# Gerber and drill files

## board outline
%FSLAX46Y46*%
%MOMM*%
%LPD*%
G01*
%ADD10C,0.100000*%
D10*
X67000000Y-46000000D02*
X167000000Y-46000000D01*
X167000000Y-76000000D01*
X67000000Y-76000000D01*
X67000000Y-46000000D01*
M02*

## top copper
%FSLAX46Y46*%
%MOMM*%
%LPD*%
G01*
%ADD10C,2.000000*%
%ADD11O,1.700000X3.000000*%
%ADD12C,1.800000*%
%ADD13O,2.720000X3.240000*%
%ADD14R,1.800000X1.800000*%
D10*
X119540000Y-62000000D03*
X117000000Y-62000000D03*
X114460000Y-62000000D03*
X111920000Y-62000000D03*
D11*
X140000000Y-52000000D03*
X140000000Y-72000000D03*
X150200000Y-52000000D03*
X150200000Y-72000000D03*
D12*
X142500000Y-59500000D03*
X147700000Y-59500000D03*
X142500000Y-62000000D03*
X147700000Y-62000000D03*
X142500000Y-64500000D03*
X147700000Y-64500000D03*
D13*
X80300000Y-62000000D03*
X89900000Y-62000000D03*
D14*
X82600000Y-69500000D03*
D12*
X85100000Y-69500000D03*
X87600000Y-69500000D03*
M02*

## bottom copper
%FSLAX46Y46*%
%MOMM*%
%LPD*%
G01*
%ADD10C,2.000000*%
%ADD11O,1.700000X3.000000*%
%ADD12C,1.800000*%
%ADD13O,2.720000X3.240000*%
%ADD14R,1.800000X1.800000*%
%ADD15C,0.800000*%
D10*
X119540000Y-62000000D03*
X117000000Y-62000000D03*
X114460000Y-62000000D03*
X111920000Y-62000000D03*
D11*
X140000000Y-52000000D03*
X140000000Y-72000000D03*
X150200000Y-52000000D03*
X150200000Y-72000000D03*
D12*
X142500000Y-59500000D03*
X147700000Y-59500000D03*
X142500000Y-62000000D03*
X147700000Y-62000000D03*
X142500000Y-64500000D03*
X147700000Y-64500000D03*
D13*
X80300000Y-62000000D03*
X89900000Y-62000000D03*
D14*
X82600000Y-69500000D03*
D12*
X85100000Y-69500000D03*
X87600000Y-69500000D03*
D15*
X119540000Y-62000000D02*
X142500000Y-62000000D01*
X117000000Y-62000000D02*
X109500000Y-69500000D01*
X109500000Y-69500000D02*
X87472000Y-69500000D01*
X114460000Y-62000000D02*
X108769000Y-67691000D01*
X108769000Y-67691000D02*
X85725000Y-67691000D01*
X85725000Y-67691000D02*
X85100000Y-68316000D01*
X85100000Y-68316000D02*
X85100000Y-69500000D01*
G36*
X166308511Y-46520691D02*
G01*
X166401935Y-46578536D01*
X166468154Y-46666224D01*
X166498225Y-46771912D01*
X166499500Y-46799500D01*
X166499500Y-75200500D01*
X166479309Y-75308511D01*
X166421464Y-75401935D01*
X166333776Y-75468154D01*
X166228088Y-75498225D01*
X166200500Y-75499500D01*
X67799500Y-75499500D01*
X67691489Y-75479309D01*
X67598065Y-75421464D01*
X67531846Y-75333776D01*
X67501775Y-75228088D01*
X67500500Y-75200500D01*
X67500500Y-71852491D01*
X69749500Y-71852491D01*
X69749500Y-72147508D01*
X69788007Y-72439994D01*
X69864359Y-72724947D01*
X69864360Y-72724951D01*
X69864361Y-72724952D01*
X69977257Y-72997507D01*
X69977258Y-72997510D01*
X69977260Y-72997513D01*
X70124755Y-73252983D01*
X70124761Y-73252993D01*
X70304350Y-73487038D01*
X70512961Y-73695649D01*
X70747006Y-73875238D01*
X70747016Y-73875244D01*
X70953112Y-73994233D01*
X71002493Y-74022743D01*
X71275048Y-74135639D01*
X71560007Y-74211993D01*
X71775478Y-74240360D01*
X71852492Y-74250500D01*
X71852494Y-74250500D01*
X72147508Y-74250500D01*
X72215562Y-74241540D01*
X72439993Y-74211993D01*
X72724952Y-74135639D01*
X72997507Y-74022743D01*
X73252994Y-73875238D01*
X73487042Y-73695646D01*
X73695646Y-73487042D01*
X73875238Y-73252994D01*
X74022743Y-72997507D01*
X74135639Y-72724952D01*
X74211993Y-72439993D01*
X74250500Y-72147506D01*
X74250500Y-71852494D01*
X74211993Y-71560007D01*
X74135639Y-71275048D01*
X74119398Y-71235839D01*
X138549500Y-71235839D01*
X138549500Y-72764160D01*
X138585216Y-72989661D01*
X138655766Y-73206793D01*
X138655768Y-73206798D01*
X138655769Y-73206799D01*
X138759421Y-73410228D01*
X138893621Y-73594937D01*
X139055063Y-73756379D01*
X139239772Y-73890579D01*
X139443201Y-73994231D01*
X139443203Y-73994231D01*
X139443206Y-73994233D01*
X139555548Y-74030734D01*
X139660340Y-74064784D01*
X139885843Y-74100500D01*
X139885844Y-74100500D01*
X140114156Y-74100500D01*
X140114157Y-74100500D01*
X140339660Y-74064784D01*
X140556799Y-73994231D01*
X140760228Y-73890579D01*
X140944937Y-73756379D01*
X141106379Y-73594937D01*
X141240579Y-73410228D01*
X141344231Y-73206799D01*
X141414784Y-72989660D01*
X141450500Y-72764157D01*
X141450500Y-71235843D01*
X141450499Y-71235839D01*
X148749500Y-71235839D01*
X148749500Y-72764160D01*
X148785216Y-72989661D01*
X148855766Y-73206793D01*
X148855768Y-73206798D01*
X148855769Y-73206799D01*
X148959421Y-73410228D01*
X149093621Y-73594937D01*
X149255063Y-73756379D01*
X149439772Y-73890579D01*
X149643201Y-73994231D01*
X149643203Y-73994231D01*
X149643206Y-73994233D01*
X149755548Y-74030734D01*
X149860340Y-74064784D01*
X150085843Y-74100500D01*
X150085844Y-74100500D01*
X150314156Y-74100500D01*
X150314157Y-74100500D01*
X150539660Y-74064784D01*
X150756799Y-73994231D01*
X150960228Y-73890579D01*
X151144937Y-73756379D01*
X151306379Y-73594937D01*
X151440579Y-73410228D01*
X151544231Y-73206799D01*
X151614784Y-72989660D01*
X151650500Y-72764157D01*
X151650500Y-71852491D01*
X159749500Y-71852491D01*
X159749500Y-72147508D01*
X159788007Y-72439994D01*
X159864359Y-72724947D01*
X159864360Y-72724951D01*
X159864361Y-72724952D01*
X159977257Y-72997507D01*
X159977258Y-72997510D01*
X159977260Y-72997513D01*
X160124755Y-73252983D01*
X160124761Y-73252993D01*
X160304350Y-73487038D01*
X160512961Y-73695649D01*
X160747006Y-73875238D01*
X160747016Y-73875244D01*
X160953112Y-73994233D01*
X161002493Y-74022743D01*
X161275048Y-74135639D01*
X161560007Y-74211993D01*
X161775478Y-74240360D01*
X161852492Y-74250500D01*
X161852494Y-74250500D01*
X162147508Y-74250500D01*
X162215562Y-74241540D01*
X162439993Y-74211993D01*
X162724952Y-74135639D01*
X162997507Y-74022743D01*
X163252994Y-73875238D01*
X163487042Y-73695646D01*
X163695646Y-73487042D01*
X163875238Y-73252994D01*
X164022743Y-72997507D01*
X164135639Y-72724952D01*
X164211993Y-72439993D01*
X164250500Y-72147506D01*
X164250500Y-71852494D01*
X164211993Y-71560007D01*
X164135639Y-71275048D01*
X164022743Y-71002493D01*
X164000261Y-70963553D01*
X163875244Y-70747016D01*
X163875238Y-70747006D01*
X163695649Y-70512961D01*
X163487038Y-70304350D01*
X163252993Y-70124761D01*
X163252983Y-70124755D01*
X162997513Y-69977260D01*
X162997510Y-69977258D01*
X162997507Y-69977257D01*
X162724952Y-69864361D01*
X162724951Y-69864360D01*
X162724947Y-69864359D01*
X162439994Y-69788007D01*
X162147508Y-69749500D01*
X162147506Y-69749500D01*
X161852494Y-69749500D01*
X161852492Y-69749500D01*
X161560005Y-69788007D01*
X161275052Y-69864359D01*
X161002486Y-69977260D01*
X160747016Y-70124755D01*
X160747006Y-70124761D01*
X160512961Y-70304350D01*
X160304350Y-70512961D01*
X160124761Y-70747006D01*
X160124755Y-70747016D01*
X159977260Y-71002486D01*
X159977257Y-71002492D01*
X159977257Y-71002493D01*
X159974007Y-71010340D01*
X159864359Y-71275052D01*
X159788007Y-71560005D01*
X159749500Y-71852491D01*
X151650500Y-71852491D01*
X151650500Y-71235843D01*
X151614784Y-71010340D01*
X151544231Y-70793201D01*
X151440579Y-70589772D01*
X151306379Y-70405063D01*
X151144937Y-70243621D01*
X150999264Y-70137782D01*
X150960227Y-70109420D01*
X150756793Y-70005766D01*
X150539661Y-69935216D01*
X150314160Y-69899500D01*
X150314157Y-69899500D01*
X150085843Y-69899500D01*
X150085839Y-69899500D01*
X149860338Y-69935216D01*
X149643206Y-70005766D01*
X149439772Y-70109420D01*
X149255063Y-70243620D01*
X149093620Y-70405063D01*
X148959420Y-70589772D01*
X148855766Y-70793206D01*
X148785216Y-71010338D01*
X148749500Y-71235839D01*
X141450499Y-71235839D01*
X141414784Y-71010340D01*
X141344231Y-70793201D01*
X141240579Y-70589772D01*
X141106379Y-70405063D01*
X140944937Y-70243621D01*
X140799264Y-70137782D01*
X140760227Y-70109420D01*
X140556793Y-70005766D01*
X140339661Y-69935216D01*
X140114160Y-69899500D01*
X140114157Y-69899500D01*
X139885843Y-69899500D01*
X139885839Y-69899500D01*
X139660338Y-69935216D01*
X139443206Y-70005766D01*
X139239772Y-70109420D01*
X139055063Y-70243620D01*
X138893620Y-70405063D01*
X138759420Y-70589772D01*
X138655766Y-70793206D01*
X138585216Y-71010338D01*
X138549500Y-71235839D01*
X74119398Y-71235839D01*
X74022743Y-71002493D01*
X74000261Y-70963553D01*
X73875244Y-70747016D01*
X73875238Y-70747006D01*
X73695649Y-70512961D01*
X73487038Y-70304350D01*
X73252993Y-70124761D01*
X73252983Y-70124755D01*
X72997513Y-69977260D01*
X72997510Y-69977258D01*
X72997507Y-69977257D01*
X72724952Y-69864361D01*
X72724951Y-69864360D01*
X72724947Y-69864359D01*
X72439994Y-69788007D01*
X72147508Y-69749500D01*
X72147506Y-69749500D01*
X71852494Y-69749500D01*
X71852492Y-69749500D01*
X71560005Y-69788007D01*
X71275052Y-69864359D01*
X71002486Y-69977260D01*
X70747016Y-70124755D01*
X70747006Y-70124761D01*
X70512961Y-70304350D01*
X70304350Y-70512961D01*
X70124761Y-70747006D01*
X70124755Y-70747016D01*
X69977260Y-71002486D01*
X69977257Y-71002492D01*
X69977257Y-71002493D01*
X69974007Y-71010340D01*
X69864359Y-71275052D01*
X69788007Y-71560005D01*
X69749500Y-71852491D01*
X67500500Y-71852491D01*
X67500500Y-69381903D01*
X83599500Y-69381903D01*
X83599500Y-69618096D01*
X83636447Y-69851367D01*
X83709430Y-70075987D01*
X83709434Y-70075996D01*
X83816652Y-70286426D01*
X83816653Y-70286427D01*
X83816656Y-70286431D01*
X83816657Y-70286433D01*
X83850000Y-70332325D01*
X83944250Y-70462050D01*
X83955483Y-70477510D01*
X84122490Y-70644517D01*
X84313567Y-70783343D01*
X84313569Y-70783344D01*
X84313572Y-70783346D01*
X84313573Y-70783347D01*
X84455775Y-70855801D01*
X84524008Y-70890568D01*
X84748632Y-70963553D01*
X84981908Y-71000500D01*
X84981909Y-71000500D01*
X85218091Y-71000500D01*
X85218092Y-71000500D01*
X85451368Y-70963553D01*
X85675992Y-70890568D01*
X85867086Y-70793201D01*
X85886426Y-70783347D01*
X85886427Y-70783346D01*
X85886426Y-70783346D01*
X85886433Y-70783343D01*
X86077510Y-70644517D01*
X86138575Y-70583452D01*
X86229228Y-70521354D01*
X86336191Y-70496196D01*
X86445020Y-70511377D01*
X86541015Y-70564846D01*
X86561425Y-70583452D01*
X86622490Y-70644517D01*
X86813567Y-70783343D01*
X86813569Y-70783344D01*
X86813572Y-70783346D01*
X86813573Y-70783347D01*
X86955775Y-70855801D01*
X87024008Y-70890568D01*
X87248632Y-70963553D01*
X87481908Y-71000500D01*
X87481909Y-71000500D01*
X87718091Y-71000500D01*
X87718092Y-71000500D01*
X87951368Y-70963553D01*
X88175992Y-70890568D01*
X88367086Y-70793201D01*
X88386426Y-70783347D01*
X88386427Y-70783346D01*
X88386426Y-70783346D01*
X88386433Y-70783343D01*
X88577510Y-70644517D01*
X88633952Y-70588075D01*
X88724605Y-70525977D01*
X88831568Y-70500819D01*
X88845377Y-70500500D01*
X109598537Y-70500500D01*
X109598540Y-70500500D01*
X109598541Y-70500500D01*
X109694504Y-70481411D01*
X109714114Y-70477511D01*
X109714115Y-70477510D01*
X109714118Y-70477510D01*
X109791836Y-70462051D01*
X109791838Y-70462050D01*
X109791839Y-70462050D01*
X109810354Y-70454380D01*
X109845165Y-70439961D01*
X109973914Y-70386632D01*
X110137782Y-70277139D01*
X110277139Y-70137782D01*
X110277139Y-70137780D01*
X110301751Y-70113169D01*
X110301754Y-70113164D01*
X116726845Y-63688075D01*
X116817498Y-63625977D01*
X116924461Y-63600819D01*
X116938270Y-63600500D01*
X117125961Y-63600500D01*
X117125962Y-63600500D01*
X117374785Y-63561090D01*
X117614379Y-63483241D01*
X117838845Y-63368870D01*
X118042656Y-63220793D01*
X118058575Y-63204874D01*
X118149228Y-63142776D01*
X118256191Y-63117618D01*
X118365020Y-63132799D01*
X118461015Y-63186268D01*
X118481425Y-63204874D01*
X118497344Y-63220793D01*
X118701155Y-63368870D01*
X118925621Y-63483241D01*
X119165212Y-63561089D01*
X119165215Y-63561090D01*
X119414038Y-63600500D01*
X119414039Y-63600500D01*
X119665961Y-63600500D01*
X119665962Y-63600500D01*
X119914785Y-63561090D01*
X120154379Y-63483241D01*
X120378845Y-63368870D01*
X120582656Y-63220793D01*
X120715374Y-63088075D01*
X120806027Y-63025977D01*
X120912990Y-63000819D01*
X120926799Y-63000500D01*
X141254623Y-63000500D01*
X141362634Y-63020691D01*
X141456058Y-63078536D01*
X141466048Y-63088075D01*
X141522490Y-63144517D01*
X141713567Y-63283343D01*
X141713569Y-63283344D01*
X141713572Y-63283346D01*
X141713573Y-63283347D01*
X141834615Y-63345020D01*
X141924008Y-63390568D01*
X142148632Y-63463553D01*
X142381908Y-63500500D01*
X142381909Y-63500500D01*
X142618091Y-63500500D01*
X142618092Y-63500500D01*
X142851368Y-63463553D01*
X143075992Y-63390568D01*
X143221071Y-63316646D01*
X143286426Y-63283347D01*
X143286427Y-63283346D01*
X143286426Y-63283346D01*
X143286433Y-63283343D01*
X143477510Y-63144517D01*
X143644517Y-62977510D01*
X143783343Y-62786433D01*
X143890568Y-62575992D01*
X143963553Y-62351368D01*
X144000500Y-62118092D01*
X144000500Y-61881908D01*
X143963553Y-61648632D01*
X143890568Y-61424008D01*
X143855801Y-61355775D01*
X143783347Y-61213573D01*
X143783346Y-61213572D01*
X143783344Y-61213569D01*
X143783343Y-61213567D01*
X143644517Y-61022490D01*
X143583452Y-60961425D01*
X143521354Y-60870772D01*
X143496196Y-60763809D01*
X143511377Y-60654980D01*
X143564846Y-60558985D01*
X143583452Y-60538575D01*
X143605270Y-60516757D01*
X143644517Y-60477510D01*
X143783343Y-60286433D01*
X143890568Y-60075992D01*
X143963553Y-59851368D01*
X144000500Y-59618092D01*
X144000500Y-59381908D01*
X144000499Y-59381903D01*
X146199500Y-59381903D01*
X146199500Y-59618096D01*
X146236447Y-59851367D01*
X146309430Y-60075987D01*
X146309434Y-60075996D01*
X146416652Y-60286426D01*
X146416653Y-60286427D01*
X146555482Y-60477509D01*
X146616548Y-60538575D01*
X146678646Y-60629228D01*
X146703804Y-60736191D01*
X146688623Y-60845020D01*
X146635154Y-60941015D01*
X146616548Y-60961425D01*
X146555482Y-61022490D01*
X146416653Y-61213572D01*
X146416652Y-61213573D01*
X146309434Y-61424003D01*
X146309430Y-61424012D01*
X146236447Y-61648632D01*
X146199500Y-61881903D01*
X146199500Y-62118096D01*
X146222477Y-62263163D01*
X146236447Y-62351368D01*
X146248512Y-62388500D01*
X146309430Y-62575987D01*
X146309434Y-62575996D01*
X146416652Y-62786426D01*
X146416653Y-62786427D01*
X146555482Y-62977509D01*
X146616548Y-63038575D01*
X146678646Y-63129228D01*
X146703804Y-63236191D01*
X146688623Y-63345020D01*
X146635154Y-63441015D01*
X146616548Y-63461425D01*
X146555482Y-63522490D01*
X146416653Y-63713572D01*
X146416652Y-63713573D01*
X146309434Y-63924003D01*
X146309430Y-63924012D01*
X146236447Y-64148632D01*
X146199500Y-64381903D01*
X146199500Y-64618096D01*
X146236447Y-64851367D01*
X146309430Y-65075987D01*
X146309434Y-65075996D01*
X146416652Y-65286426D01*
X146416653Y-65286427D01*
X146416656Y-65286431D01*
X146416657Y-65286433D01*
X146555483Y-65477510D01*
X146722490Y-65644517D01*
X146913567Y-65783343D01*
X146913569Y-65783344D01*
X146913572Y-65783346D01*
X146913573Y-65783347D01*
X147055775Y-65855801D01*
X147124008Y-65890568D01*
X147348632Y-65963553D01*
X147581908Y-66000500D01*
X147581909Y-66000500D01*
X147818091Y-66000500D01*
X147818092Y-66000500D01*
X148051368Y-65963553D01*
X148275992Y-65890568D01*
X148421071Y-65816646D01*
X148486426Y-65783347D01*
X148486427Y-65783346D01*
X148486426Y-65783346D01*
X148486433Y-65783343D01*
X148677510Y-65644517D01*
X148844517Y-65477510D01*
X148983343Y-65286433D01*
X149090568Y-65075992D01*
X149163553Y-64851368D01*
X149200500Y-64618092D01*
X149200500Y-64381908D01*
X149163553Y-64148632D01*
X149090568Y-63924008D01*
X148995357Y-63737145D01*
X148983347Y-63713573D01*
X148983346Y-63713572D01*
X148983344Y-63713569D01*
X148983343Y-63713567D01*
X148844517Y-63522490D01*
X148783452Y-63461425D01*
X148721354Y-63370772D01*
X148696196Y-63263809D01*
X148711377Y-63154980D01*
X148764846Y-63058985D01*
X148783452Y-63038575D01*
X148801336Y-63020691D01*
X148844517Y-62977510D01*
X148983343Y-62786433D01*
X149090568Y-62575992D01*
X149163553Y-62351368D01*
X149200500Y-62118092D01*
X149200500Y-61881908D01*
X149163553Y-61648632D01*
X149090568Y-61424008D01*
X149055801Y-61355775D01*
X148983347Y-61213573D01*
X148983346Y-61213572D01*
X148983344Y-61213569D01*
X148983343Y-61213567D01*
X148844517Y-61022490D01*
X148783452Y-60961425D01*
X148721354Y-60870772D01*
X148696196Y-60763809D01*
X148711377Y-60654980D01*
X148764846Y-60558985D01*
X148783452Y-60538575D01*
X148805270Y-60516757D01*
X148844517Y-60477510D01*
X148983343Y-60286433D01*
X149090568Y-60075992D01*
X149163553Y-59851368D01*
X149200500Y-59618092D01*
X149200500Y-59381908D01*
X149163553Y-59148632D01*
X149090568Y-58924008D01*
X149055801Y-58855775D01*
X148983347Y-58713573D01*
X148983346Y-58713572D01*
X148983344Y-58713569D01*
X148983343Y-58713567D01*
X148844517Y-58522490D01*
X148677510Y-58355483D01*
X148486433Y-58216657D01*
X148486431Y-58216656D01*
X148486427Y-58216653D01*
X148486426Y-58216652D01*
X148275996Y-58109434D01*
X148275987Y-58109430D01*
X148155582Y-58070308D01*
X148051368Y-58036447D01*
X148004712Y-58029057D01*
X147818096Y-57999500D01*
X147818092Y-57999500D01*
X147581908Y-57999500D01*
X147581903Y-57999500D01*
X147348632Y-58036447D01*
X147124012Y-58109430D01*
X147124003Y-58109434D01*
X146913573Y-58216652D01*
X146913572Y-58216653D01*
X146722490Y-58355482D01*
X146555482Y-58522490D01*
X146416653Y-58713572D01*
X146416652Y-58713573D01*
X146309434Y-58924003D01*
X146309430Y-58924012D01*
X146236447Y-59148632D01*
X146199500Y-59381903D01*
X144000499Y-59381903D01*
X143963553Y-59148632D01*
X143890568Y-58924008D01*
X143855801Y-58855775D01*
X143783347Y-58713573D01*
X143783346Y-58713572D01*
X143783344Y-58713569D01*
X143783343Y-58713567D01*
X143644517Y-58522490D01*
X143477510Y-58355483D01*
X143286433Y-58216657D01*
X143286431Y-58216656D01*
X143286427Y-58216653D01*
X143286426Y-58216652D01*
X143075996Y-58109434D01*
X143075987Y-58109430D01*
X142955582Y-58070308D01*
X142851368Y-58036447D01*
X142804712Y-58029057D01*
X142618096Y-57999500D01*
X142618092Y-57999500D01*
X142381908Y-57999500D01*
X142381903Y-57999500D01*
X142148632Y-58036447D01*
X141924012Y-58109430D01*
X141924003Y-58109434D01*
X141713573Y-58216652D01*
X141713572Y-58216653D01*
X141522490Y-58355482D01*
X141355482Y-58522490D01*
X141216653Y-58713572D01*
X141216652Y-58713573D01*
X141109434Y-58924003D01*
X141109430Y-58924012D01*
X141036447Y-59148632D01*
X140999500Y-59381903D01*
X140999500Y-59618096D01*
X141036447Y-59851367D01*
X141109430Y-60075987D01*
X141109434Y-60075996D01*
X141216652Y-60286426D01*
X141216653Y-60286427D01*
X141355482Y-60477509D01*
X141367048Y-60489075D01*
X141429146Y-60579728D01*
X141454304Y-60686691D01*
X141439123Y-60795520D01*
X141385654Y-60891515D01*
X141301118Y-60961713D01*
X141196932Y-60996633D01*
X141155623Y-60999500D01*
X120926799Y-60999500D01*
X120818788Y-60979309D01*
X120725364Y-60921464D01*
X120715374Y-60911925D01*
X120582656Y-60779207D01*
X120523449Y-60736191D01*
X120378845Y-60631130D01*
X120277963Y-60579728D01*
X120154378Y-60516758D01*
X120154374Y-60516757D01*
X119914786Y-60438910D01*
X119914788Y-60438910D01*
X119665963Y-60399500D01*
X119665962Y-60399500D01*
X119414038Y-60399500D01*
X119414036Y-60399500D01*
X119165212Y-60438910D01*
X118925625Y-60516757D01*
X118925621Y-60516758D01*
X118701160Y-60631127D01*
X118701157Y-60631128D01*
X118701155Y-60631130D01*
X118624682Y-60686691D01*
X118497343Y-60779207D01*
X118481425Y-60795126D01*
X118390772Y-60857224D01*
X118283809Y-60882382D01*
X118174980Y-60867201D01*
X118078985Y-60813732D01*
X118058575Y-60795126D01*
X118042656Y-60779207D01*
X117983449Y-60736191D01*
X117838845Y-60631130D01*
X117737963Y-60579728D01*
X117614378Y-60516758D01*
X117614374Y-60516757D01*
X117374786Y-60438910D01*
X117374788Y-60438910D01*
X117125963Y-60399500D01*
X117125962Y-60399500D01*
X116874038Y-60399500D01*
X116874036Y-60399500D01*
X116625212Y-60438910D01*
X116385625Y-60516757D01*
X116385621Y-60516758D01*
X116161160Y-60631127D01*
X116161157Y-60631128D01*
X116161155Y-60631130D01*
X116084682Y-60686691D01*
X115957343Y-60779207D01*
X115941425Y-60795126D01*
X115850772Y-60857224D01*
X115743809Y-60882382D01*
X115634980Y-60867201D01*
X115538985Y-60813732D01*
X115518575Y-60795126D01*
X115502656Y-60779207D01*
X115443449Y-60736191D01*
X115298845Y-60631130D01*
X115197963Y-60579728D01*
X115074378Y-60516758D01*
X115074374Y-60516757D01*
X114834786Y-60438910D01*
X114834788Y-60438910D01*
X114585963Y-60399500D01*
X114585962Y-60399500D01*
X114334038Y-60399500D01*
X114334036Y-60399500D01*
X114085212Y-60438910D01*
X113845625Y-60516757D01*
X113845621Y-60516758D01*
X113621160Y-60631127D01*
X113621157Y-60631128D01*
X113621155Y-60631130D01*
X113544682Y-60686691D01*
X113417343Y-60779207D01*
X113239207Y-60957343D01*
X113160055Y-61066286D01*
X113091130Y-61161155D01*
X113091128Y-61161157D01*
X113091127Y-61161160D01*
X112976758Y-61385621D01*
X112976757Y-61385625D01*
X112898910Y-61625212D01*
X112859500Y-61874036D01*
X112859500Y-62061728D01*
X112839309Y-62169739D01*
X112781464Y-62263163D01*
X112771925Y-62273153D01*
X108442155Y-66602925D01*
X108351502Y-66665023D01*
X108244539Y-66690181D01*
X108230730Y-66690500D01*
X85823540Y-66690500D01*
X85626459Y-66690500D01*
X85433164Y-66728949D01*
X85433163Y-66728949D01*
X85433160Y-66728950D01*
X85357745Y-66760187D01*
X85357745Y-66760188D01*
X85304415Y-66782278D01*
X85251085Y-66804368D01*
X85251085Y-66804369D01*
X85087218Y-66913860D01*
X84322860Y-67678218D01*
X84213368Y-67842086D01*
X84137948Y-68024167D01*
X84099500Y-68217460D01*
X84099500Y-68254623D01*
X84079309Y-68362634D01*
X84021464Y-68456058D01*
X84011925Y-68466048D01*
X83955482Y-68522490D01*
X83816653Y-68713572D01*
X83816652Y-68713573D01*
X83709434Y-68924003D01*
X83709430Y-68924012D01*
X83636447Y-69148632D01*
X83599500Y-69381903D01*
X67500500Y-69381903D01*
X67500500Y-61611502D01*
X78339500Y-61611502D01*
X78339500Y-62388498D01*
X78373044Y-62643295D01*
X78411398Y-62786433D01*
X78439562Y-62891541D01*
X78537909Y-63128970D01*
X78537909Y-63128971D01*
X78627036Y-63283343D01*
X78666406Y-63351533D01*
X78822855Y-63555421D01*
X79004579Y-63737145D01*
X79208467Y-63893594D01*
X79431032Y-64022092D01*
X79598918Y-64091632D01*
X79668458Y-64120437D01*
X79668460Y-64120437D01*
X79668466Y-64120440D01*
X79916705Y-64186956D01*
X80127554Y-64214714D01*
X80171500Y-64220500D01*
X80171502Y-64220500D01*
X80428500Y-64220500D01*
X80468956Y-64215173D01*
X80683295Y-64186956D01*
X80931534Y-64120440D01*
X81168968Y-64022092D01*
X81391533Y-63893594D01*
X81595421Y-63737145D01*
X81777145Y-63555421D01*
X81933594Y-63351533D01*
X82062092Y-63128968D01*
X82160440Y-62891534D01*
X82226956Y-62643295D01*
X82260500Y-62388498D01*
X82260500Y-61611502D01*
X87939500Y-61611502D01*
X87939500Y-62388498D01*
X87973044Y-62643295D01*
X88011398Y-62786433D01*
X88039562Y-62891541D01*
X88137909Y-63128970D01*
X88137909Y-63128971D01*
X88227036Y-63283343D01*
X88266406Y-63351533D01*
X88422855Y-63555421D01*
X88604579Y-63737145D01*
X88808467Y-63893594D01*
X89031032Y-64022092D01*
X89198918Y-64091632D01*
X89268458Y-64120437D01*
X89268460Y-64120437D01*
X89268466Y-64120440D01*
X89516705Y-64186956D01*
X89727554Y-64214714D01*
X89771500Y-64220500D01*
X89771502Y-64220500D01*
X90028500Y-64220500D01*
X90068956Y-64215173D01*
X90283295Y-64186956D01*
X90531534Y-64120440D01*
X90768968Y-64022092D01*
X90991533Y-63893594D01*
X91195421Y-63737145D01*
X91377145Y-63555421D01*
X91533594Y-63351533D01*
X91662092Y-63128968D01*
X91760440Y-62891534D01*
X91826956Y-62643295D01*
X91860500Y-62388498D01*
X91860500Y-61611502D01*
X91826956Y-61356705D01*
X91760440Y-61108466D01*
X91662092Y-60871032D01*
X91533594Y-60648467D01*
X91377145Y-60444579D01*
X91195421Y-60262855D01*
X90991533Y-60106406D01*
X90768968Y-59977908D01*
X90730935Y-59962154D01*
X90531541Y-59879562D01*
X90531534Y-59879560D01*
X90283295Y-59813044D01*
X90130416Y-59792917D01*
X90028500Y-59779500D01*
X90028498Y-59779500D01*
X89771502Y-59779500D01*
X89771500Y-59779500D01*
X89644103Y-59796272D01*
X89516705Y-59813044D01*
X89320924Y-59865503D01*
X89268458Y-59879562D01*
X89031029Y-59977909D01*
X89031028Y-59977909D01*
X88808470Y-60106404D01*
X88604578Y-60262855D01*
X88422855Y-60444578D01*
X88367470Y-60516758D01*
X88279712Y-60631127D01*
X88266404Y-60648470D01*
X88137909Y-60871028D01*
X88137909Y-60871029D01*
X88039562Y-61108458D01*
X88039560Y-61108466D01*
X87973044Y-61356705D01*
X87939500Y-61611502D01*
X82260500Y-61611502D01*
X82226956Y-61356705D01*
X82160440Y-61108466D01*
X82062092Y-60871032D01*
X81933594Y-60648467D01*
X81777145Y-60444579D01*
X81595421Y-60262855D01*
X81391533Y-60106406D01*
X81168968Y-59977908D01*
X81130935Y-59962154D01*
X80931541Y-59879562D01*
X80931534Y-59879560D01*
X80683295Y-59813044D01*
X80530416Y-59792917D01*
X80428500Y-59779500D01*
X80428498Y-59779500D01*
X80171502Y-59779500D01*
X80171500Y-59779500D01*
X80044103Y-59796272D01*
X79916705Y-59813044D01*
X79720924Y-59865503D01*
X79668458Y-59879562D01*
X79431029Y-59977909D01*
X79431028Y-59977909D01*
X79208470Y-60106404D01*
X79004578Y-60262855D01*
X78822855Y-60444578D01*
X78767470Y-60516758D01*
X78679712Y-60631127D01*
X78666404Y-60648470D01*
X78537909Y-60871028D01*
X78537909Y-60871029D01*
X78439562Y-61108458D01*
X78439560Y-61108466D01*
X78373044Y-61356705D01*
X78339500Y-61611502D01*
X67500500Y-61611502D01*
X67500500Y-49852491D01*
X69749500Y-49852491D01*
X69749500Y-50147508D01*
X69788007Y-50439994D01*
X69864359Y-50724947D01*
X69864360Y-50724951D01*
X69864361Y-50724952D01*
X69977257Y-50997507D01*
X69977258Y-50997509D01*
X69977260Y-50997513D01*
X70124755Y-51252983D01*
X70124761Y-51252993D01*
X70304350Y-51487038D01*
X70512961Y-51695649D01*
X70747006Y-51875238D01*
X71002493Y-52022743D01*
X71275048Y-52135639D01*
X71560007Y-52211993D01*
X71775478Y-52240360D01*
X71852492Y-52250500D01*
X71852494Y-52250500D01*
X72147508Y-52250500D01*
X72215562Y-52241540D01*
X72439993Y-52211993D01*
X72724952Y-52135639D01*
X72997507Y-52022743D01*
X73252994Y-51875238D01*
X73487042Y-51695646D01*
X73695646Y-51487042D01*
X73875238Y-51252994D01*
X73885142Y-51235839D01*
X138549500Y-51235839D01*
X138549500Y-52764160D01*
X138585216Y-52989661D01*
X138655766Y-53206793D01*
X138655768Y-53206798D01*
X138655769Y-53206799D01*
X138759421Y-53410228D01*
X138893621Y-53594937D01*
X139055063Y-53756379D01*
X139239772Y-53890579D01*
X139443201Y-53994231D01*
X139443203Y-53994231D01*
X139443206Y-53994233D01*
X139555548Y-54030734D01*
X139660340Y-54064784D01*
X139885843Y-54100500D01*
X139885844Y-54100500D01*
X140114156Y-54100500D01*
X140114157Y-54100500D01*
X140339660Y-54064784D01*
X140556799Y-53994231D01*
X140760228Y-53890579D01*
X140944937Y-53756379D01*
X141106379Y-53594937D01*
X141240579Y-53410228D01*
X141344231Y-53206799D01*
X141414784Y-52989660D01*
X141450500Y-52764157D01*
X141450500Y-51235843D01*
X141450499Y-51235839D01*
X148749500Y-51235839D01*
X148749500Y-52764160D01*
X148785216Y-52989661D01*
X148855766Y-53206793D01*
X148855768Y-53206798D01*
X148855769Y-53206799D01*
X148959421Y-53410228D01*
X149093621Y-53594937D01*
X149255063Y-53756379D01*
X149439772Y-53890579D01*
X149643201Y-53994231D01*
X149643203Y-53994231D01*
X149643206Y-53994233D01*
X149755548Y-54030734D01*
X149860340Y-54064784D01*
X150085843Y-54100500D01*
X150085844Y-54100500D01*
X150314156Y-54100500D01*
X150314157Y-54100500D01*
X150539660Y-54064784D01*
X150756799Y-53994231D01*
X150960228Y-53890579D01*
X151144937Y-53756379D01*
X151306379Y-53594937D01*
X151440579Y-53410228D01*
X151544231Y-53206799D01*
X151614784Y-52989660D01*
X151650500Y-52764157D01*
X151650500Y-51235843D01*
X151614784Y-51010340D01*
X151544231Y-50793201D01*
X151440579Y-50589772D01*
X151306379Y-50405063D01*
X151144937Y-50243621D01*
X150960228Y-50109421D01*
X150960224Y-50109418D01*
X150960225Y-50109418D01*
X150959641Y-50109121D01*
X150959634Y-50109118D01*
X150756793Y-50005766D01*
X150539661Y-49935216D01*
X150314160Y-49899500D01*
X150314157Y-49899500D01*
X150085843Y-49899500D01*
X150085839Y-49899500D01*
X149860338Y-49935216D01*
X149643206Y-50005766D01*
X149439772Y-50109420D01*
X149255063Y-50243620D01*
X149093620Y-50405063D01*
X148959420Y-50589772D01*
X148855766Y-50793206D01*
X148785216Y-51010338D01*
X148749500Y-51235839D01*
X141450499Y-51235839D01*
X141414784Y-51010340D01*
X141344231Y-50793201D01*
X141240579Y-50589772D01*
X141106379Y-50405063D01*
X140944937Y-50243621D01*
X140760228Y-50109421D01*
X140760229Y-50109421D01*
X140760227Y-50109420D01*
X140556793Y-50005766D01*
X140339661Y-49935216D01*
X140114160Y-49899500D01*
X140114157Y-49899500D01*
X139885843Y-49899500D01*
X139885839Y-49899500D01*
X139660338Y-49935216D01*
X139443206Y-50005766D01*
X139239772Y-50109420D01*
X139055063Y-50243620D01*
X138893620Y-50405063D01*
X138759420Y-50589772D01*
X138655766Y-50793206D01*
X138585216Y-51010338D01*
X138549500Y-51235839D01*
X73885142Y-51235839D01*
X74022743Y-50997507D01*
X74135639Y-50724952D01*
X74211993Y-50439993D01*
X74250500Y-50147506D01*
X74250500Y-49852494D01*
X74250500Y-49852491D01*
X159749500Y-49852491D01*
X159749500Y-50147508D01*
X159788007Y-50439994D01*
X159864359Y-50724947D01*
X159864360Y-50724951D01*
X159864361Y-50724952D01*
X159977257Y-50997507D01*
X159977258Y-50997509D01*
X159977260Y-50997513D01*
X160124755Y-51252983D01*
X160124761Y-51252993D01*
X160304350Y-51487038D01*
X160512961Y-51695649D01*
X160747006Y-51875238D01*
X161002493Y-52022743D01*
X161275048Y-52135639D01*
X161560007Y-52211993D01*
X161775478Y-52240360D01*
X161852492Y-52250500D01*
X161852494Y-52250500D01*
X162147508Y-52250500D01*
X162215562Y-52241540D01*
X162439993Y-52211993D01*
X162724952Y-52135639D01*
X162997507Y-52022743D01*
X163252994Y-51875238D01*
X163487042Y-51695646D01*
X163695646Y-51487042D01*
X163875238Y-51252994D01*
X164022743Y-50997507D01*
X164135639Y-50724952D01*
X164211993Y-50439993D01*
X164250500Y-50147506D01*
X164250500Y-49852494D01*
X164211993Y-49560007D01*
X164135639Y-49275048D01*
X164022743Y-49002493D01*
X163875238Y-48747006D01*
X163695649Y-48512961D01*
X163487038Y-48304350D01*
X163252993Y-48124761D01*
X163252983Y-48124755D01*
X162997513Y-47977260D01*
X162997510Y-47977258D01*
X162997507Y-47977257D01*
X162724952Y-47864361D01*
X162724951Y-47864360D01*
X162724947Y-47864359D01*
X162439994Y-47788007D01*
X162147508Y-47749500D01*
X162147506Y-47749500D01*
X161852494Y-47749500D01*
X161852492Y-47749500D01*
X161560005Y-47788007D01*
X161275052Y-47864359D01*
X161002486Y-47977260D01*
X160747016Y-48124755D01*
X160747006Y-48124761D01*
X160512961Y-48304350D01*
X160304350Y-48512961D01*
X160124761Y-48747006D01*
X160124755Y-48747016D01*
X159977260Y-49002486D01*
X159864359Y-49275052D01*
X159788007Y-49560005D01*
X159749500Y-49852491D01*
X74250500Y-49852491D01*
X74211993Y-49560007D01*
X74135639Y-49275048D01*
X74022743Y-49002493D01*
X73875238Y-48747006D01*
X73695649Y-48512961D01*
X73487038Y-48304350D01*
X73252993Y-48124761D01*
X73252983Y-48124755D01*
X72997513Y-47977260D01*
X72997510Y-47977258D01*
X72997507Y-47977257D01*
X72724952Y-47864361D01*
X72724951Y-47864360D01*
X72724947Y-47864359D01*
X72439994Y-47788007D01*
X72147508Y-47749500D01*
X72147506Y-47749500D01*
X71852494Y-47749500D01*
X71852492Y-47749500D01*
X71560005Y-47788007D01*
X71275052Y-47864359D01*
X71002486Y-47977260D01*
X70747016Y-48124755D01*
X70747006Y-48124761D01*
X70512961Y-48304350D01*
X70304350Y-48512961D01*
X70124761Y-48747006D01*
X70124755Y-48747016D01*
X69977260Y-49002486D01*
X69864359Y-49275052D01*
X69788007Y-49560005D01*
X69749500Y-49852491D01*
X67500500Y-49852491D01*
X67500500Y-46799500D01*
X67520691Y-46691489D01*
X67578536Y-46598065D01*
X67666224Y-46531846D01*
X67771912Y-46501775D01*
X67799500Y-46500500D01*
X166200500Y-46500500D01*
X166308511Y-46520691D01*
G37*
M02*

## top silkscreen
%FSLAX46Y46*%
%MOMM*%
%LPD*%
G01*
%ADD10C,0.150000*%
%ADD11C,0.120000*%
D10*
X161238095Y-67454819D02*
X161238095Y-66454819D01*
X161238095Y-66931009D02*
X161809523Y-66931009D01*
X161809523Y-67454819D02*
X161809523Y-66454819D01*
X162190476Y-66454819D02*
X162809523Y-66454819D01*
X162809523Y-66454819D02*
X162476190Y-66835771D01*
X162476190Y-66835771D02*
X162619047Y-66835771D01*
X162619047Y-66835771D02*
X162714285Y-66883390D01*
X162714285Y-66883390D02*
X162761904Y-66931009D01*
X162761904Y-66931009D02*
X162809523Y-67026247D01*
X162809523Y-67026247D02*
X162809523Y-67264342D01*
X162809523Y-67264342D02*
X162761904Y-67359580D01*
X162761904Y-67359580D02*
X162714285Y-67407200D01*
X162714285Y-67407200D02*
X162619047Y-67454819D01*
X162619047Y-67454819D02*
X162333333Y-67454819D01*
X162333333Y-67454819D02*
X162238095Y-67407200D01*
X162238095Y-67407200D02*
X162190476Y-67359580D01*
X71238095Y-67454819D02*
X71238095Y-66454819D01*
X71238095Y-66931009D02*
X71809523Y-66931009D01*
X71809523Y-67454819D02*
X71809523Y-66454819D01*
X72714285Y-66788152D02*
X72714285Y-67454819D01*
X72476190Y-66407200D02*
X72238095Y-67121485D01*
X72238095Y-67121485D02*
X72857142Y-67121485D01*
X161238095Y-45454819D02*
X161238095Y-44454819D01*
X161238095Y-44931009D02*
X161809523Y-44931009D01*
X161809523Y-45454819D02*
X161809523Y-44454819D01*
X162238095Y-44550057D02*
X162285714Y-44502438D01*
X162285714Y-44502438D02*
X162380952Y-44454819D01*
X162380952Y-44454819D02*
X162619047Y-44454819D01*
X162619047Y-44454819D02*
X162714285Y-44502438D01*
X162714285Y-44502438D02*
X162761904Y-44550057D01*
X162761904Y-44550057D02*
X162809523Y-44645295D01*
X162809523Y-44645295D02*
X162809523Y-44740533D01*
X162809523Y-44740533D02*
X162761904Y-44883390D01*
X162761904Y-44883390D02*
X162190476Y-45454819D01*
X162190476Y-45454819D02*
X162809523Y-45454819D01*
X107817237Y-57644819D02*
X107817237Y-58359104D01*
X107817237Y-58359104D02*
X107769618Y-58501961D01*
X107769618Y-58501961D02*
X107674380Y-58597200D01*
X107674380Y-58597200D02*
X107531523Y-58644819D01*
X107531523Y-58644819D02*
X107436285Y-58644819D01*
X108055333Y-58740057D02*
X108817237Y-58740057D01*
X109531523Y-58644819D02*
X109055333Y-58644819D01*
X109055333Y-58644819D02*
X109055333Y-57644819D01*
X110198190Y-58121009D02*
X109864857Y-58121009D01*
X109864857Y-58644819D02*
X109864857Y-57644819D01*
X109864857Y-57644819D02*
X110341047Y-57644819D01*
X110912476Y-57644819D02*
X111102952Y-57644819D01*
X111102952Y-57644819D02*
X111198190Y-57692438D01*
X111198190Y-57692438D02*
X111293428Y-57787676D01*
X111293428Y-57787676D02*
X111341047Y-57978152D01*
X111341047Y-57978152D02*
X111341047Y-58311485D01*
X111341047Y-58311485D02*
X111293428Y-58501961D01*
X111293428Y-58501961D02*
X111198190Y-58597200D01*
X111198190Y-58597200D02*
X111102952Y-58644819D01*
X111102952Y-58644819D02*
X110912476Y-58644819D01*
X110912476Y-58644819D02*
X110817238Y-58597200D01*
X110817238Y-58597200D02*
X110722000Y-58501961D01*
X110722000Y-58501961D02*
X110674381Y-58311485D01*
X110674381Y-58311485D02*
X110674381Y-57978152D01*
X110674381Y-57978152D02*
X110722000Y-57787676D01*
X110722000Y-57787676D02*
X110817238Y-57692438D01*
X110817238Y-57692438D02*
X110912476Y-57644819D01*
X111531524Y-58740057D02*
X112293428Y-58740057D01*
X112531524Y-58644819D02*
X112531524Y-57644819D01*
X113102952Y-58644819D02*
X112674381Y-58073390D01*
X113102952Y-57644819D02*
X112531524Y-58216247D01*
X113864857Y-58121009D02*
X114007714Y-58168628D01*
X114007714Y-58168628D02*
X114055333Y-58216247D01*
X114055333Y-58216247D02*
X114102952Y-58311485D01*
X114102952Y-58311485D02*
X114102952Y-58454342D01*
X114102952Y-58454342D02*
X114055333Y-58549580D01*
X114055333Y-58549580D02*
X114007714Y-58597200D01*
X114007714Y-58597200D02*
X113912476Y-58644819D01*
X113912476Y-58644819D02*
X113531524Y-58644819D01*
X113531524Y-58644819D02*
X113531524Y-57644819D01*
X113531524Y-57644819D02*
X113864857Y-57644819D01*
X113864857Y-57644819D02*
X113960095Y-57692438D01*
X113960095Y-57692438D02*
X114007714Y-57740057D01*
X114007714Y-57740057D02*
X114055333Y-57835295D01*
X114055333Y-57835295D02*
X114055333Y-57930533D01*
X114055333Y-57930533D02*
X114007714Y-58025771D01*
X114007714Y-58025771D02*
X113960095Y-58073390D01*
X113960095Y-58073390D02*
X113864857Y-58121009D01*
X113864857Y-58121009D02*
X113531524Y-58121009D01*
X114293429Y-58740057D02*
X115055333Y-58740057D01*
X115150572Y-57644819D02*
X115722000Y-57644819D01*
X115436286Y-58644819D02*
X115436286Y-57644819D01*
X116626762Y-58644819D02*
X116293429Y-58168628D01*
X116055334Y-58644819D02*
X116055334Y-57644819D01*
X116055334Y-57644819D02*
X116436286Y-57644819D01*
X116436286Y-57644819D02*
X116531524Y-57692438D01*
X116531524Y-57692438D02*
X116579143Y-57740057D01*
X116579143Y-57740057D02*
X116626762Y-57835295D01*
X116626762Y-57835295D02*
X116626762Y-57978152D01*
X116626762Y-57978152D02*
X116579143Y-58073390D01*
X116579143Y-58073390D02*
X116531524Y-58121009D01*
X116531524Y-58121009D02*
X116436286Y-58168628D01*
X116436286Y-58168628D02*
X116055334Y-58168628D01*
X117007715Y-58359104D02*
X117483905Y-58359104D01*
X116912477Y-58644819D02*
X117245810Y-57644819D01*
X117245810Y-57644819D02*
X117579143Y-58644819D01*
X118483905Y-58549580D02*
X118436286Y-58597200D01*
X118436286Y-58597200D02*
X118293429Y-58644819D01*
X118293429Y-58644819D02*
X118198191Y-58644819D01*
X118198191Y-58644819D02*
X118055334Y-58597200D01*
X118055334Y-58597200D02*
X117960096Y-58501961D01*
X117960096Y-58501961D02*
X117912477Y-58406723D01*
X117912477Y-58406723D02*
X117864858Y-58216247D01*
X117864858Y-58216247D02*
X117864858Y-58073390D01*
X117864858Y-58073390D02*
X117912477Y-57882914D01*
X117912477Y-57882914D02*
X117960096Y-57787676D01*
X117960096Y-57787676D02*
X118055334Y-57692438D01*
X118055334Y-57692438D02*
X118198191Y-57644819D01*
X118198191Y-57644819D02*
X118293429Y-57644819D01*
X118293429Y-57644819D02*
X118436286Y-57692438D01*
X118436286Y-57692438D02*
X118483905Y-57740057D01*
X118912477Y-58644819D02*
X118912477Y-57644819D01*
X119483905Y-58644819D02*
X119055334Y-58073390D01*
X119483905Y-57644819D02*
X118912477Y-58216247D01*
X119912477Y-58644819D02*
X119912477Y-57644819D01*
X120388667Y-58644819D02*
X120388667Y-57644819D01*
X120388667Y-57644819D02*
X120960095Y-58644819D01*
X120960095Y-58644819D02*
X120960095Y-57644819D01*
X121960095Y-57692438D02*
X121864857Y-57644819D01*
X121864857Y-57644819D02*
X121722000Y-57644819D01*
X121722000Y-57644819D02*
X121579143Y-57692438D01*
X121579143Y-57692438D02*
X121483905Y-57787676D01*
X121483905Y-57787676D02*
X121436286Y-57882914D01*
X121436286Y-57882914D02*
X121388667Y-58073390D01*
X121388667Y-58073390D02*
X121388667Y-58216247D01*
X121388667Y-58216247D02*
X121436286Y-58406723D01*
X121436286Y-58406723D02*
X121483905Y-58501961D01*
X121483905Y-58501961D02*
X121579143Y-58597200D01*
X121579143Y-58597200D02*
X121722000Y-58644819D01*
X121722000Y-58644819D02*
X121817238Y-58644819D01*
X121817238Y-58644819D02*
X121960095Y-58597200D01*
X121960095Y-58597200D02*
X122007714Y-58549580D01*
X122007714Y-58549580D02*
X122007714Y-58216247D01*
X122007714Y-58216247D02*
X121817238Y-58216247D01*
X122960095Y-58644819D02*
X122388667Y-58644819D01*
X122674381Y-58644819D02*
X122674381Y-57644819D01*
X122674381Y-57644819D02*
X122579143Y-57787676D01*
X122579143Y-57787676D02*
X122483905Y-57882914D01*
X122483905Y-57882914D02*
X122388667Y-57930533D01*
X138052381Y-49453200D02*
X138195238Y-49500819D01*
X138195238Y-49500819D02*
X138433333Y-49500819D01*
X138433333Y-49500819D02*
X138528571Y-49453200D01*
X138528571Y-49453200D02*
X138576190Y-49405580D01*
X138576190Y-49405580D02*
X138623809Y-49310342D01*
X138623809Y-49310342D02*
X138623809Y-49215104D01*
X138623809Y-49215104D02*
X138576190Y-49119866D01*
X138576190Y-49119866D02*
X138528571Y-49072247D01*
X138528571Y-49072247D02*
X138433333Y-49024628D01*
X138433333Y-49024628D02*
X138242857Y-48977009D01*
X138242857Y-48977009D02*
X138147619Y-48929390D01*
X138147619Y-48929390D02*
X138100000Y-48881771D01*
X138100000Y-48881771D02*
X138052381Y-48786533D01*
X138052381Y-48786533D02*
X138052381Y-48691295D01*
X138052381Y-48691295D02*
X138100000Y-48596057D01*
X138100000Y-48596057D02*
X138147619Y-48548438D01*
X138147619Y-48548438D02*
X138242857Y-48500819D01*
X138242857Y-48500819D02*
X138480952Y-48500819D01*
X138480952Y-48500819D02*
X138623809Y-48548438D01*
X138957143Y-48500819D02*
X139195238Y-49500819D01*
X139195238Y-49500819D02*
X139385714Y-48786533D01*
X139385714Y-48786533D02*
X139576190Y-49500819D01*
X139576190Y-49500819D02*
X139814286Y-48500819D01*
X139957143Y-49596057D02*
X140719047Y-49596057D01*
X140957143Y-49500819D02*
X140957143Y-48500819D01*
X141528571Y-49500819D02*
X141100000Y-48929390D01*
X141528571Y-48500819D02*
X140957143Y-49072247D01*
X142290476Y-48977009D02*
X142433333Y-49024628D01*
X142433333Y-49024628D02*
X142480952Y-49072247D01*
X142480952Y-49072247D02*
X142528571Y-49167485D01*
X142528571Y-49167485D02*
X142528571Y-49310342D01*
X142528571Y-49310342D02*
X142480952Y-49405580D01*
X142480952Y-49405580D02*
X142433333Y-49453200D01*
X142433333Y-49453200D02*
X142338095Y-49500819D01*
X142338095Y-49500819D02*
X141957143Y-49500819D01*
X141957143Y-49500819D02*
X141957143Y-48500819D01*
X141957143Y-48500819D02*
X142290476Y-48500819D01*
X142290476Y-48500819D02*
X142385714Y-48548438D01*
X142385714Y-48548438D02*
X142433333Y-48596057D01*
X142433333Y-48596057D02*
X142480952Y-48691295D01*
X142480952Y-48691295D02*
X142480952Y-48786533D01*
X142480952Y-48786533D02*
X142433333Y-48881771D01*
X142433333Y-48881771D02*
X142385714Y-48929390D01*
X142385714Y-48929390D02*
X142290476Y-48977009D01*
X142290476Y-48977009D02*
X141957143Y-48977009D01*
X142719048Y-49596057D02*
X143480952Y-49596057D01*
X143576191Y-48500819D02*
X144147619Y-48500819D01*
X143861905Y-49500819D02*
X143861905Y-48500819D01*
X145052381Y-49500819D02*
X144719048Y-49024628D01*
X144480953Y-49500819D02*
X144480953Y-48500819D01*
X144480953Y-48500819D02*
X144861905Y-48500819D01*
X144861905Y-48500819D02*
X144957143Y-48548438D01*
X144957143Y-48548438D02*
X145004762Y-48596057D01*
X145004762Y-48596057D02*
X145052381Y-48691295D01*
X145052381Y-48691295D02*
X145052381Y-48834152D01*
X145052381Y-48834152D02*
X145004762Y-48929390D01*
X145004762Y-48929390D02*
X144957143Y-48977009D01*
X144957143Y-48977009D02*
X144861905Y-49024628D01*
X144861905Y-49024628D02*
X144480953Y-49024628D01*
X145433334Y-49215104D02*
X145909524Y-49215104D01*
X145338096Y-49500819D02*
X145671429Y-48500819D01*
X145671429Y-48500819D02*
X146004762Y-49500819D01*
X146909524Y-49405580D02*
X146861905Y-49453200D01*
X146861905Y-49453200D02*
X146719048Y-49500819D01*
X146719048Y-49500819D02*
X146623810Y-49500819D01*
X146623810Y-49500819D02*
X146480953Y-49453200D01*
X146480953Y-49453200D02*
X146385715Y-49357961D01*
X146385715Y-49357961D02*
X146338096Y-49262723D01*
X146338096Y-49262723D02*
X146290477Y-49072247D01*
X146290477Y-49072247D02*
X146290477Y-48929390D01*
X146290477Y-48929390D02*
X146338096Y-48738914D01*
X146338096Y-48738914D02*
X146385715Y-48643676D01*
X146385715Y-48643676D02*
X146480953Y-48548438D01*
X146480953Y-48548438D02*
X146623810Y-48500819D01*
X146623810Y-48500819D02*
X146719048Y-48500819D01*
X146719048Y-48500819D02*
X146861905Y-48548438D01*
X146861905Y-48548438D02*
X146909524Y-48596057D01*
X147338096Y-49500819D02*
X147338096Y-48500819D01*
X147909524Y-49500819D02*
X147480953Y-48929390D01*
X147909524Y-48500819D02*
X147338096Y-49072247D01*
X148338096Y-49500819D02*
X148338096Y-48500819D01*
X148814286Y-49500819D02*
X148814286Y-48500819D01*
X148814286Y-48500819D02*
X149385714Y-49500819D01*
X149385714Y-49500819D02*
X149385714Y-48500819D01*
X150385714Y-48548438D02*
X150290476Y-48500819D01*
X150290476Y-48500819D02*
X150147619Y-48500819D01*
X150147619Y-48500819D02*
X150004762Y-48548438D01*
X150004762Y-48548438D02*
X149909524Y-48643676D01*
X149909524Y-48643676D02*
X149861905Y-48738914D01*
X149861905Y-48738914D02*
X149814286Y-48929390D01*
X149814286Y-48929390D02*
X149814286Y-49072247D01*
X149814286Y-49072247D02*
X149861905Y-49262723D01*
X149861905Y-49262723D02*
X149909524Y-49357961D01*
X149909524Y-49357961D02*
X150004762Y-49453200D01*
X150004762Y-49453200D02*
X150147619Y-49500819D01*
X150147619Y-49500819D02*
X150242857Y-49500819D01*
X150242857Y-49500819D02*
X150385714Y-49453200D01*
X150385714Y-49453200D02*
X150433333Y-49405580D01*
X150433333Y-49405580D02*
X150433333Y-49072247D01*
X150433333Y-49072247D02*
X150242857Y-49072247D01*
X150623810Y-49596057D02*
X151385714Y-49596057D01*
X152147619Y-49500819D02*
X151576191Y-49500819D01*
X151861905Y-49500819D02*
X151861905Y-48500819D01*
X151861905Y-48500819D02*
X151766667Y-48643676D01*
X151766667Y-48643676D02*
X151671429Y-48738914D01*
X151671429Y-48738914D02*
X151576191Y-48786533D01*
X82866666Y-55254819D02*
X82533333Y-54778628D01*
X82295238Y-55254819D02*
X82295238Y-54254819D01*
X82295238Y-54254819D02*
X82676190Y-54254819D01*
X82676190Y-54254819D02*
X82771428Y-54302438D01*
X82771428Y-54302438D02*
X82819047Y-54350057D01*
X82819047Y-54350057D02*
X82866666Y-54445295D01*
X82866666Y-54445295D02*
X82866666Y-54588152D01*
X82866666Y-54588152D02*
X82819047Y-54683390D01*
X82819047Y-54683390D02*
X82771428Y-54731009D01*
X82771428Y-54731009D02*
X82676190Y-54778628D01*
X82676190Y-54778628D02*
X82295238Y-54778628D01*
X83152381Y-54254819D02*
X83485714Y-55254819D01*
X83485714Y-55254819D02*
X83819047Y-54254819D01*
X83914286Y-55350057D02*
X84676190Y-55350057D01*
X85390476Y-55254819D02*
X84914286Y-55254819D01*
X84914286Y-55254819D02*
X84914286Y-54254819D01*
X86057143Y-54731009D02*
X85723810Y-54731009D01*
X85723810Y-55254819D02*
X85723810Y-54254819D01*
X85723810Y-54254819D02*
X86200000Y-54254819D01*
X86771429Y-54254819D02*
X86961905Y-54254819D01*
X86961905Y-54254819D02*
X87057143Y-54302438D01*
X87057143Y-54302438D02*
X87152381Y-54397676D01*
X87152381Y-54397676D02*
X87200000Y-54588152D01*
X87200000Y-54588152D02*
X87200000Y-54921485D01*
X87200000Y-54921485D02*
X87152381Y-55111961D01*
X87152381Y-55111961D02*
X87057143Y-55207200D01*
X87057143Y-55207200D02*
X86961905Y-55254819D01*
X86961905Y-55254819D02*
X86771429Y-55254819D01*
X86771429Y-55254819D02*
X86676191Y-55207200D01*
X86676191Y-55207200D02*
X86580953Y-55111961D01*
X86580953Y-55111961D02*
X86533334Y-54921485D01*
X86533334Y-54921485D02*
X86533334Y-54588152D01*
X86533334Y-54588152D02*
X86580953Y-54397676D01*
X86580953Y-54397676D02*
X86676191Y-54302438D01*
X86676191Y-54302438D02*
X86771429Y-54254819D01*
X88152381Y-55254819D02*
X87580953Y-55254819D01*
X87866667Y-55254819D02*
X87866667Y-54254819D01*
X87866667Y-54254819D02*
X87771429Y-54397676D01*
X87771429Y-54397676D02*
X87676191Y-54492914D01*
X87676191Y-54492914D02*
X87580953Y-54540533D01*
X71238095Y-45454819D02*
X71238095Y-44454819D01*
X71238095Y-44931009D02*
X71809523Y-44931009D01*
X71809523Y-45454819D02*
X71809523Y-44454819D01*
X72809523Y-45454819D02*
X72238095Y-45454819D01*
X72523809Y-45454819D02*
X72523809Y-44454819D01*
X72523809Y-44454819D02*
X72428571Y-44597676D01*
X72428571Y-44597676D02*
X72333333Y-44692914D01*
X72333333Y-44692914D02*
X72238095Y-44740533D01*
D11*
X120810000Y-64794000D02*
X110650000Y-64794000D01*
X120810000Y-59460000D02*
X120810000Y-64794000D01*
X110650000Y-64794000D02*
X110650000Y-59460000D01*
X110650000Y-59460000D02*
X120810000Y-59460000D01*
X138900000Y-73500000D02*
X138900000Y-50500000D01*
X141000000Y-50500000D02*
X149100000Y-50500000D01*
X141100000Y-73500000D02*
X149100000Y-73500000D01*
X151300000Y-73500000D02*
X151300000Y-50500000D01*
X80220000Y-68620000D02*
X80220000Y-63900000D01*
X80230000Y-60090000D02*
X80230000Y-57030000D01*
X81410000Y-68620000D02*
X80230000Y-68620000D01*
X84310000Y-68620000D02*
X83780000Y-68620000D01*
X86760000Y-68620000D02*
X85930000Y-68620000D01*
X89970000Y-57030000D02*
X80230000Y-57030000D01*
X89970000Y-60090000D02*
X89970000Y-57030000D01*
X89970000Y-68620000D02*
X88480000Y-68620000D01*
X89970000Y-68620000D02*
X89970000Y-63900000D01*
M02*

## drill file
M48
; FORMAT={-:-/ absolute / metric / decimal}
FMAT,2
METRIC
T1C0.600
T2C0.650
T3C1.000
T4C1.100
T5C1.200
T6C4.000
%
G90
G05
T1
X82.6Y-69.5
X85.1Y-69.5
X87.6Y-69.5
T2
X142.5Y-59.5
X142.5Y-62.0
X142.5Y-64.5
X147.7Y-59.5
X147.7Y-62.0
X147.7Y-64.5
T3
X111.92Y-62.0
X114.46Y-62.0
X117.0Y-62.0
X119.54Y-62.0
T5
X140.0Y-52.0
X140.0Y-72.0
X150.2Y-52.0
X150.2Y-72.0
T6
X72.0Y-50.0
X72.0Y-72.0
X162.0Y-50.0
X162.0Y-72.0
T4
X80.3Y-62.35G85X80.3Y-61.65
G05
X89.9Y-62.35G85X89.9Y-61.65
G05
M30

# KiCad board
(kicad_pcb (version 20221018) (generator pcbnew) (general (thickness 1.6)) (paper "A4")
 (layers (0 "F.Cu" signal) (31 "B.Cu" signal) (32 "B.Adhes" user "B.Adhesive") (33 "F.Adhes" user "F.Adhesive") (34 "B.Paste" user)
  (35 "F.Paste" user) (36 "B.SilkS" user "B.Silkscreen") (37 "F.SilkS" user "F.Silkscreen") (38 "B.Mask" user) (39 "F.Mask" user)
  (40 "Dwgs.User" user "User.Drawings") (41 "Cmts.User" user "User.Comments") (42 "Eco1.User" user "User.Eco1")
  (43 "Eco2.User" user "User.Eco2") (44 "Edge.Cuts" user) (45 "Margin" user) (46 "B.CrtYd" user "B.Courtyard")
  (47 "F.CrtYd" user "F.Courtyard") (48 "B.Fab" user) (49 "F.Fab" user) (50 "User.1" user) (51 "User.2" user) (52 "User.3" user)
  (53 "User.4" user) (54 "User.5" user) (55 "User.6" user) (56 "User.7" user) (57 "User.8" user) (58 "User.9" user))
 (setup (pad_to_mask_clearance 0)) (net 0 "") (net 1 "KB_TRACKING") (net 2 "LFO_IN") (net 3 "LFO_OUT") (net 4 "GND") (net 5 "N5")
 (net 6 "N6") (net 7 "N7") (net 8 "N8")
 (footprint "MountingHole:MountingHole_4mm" (layer "F.Cu") (at 162 72)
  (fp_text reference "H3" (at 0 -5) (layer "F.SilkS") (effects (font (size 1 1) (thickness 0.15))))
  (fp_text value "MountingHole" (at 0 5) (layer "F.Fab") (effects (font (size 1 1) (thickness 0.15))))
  (pad "" np_thru_hole circle (at 0 0) (size 4 4) (drill 4) (layers "*.Cu" "*.Mask")))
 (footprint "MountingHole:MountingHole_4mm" (layer "F.Cu") (at 72 72)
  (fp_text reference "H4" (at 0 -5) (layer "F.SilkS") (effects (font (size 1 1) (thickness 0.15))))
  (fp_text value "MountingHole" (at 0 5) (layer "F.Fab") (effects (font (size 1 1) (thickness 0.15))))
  (pad "" np_thru_hole circle (at 0 0) (size 4 4) (drill 4) (layers "*.Cu" "*.Mask")))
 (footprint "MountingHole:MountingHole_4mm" (layer "F.Cu") (at 162 50)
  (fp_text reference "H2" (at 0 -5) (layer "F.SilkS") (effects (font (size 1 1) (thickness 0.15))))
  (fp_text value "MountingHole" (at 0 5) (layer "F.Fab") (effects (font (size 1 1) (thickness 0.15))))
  (pad "" np_thru_hole circle (at 0 0) (size 4 4) (drill 4) (layers "*.Cu" "*.Mask")))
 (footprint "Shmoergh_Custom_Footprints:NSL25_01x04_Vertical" (layer "F.Cu") (at 119.54 62 180)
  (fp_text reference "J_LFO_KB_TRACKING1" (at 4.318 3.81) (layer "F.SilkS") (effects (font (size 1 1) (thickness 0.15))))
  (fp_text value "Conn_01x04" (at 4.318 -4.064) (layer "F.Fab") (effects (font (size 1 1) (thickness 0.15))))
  (fp_line (start -1.27 -2.794) (end 8.89 -2.794) (stroke (width 0.12) (type solid)) (layer "F.SilkS"))
  (fp_line (start -1.27 2.54) (end -1.27 -2.794) (stroke (width 0.12) (type solid)) (layer "F.SilkS"))
  (fp_line (start 8.89 -2.794) (end 8.89 2.54) (stroke (width 0.12) (type solid)) (layer "F.SilkS"))
  (fp_line (start 8.89 2.54) (end -1.27 2.54) (stroke (width 0.12) (type solid)) (layer "F.SilkS"))
  (pad "1" thru_hole circle (at 0 0 180) (size 2 2) (drill 1) (layers "*.Cu" "*.Mask") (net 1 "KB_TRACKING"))
  (pad "2" thru_hole circle (at 2.54 0 180) (size 2 2) (drill 1) (layers "*.Cu" "*.Mask") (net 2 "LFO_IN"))
  (pad "3" thru_hole circle (at 5.08 0 180) (size 2 2) (drill 1) (layers "*.Cu" "*.Mask") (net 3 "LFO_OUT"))
  (pad "4" thru_hole circle (at 7.62 0 180) (size 2 2) (drill 1) (layers "*.Cu" "*.Mask") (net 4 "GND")))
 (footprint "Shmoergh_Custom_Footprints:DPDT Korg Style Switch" (layer "F.Cu") (at 145.1 62)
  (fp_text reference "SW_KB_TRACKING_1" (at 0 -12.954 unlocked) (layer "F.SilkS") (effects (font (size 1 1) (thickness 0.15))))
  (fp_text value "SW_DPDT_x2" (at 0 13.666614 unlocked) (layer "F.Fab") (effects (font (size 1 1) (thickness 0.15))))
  (fp_line (start -6.2 11.5) (end -6.2 -11.5) (stroke (width 0.12) (type default)) (layer "F.SilkS"))
  (fp_line (start -4.1 -11.5) (end 4 -11.5) (stroke (width 0.12) (type default)) (layer "F.SilkS"))
  (fp_line (start -4 11.5) (end 4 11.5) (stroke (width 0.12) (type default)) (layer "F.SilkS"))
  (fp_line (start 6.2 11.5) (end 6.2 -11.5) (stroke (width 0.12) (type default)) (layer "F.SilkS"))
  (pad "" thru_hole oval (at -5.1 -10) (size 1.7 3) (drill 1.2) (layers "*.Cu" "*.Mask"))
  (pad "" thru_hole oval (at -5.1 10) (size 1.7 3) (drill 1.2) (layers "*.Cu" "*.Mask"))
  (pad "" thru_hole oval (at 5.1 -10) (size 1.7 3) (drill 1.2) (layers "*.Cu" "*.Mask"))
  (pad "" thru_hole oval (at 5.1 10) (size 1.7 3) (drill 1.2) (layers "*.Cu" "*.Mask"))
  (pad "1" thru_hole circle (at -2.6 -2.5) (size 1.8 1.8) (drill 0.65) (layers "*.Cu" "*.Mask") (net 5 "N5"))
  (pad "2" thru_hole circle (at 2.6 -2.5) (size 1.8 1.8) (drill 0.65) (layers "*.Cu" "*.Mask") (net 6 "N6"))
  (pad "3" thru_hole circle (at -2.6 0) (size 1.8 1.8) (drill 0.65) (layers "*.Cu" "*.Mask") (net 1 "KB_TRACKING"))
  (pad "4" thru_hole circle (at 2.6 0) (size 1.8 1.8) (drill 0.65) (layers "*.Cu" "*.Mask") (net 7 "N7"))
  (pad "5" thru_hole circle (at -2.6 2.5) (size 1.8 1.8) (drill 0.65) (layers "*.Cu" "*.Mask") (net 4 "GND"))
  (pad "6" thru_hole circle (at 2.6 2.5) (size 1.8 1.8) (drill 0.65) (layers "*.Cu" "*.Mask") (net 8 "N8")))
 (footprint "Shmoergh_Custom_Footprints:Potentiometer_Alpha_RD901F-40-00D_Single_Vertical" (layer "F.Cu") (at 85.1 62)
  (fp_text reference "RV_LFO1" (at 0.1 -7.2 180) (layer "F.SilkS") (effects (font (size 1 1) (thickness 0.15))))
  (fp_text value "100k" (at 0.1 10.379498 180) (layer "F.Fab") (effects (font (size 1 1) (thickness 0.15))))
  (fp_line (start -4.88 6.62) (end -4.88 1.9) (stroke (width 0.12) (type solid)) (layer "F.SilkS"))
  (fp_line (start -4.87 -1.91) (end -4.87 -4.97) (stroke (width 0.12) (type solid)) (layer "F.SilkS"))
  (fp_line (start -3.69 6.62) (end -4.87 6.62) (stroke (width 0.12) (type solid)) (layer "F.SilkS"))
  (fp_line (start -0.79 6.62) (end -1.32 6.62) (stroke (width 0.12) (type solid)) (layer "F.SilkS"))
  (fp_line (start 1.66 6.62) (end 0.83 6.62) (stroke (width 0.12) (type solid)) (layer "F.SilkS"))
  (fp_line (start 4.87 -4.97) (end -4.87 -4.97) (stroke (width 0.12) (type solid)) (layer "F.SilkS"))
  (fp_line (start 4.87 -1.91) (end 4.87 -4.97) (stroke (width 0.12) (type solid)) (layer "F.SilkS"))
  (fp_line (start 4.87 6.62) (end 3.38 6.62) (stroke (width 0.12) (type solid)) (layer "F.SilkS"))
  (fp_line (start 4.87 6.62) (end 4.87 1.9) (stroke (width 0.12) (type solid)) (layer "F.SilkS"))
  (pad "" thru_hole oval (at -4.8 0 180) (size 2.72 3.24) (drill oval 1.1 1.8) (layers "*.Cu" "*.Mask"))
  (pad "" thru_hole oval (at 4.8 0 180) (size 2.72 3.24) (drill oval 1.1 1.8) (layers "*.Cu" "*.Mask"))
  (pad "1" thru_hole rect (at -2.5 7.5 180) (size 1.8 1.8) (drill 0.6) (layers "*.Cu" "*.Mask") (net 4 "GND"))
  (pad "2" thru_hole circle (at 0 7.5 180) (size 1.8 1.8) (drill 0.6) (layers "*.Cu" "*.Mask") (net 3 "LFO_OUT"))
  (pad "3" thru_hole circle (at 2.5 7.5 180) (size 1.8 1.8) (drill 0.6) (layers "*.Cu" "*.Mask") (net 2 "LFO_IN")))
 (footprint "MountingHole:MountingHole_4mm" (layer "F.Cu") (at 72 50)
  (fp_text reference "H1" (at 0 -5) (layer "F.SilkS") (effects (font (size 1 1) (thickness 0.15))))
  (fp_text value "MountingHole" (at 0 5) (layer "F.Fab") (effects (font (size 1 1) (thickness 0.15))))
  (pad "" np_thru_hole circle (at 0 0) (size 4 4) (drill 4) (layers "*.Cu" "*.Mask")))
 (gr_rect (start 67 46) (end 167 76) (stroke (width 0.1) (type default)) (fill none) (layer "Edge.Cuts"))
 (segment (start 119.54 62) (end 142.5 62) (width 0.8) (layer "B.Cu") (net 1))
 (segment (start 117 62) (end 109.5 69.5) (width 0.8) (layer "B.Cu") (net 2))
 (segment (start 109.5 69.5) (end 87.472 69.5) (width 0.8) (layer "B.Cu") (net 2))
 (segment (start 114.46 62) (end 108.769 67.691) (width 0.8) (layer "B.Cu") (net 3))
 (segment (start 108.769 67.691) (end 85.725 67.691) (width 0.8) (layer "B.Cu") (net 3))
 (segment (start 85.725 67.691) (end 85.1 68.316) (width 0.8) (layer "B.Cu") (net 3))
 (segment (start 85.1 68.316) (end 85.1 69.5) (width 0.8) (layer "B.Cu") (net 3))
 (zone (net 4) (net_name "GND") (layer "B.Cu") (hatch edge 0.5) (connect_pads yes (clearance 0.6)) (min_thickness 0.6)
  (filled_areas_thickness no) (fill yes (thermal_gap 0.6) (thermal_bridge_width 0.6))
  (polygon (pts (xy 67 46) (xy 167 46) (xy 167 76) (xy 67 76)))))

